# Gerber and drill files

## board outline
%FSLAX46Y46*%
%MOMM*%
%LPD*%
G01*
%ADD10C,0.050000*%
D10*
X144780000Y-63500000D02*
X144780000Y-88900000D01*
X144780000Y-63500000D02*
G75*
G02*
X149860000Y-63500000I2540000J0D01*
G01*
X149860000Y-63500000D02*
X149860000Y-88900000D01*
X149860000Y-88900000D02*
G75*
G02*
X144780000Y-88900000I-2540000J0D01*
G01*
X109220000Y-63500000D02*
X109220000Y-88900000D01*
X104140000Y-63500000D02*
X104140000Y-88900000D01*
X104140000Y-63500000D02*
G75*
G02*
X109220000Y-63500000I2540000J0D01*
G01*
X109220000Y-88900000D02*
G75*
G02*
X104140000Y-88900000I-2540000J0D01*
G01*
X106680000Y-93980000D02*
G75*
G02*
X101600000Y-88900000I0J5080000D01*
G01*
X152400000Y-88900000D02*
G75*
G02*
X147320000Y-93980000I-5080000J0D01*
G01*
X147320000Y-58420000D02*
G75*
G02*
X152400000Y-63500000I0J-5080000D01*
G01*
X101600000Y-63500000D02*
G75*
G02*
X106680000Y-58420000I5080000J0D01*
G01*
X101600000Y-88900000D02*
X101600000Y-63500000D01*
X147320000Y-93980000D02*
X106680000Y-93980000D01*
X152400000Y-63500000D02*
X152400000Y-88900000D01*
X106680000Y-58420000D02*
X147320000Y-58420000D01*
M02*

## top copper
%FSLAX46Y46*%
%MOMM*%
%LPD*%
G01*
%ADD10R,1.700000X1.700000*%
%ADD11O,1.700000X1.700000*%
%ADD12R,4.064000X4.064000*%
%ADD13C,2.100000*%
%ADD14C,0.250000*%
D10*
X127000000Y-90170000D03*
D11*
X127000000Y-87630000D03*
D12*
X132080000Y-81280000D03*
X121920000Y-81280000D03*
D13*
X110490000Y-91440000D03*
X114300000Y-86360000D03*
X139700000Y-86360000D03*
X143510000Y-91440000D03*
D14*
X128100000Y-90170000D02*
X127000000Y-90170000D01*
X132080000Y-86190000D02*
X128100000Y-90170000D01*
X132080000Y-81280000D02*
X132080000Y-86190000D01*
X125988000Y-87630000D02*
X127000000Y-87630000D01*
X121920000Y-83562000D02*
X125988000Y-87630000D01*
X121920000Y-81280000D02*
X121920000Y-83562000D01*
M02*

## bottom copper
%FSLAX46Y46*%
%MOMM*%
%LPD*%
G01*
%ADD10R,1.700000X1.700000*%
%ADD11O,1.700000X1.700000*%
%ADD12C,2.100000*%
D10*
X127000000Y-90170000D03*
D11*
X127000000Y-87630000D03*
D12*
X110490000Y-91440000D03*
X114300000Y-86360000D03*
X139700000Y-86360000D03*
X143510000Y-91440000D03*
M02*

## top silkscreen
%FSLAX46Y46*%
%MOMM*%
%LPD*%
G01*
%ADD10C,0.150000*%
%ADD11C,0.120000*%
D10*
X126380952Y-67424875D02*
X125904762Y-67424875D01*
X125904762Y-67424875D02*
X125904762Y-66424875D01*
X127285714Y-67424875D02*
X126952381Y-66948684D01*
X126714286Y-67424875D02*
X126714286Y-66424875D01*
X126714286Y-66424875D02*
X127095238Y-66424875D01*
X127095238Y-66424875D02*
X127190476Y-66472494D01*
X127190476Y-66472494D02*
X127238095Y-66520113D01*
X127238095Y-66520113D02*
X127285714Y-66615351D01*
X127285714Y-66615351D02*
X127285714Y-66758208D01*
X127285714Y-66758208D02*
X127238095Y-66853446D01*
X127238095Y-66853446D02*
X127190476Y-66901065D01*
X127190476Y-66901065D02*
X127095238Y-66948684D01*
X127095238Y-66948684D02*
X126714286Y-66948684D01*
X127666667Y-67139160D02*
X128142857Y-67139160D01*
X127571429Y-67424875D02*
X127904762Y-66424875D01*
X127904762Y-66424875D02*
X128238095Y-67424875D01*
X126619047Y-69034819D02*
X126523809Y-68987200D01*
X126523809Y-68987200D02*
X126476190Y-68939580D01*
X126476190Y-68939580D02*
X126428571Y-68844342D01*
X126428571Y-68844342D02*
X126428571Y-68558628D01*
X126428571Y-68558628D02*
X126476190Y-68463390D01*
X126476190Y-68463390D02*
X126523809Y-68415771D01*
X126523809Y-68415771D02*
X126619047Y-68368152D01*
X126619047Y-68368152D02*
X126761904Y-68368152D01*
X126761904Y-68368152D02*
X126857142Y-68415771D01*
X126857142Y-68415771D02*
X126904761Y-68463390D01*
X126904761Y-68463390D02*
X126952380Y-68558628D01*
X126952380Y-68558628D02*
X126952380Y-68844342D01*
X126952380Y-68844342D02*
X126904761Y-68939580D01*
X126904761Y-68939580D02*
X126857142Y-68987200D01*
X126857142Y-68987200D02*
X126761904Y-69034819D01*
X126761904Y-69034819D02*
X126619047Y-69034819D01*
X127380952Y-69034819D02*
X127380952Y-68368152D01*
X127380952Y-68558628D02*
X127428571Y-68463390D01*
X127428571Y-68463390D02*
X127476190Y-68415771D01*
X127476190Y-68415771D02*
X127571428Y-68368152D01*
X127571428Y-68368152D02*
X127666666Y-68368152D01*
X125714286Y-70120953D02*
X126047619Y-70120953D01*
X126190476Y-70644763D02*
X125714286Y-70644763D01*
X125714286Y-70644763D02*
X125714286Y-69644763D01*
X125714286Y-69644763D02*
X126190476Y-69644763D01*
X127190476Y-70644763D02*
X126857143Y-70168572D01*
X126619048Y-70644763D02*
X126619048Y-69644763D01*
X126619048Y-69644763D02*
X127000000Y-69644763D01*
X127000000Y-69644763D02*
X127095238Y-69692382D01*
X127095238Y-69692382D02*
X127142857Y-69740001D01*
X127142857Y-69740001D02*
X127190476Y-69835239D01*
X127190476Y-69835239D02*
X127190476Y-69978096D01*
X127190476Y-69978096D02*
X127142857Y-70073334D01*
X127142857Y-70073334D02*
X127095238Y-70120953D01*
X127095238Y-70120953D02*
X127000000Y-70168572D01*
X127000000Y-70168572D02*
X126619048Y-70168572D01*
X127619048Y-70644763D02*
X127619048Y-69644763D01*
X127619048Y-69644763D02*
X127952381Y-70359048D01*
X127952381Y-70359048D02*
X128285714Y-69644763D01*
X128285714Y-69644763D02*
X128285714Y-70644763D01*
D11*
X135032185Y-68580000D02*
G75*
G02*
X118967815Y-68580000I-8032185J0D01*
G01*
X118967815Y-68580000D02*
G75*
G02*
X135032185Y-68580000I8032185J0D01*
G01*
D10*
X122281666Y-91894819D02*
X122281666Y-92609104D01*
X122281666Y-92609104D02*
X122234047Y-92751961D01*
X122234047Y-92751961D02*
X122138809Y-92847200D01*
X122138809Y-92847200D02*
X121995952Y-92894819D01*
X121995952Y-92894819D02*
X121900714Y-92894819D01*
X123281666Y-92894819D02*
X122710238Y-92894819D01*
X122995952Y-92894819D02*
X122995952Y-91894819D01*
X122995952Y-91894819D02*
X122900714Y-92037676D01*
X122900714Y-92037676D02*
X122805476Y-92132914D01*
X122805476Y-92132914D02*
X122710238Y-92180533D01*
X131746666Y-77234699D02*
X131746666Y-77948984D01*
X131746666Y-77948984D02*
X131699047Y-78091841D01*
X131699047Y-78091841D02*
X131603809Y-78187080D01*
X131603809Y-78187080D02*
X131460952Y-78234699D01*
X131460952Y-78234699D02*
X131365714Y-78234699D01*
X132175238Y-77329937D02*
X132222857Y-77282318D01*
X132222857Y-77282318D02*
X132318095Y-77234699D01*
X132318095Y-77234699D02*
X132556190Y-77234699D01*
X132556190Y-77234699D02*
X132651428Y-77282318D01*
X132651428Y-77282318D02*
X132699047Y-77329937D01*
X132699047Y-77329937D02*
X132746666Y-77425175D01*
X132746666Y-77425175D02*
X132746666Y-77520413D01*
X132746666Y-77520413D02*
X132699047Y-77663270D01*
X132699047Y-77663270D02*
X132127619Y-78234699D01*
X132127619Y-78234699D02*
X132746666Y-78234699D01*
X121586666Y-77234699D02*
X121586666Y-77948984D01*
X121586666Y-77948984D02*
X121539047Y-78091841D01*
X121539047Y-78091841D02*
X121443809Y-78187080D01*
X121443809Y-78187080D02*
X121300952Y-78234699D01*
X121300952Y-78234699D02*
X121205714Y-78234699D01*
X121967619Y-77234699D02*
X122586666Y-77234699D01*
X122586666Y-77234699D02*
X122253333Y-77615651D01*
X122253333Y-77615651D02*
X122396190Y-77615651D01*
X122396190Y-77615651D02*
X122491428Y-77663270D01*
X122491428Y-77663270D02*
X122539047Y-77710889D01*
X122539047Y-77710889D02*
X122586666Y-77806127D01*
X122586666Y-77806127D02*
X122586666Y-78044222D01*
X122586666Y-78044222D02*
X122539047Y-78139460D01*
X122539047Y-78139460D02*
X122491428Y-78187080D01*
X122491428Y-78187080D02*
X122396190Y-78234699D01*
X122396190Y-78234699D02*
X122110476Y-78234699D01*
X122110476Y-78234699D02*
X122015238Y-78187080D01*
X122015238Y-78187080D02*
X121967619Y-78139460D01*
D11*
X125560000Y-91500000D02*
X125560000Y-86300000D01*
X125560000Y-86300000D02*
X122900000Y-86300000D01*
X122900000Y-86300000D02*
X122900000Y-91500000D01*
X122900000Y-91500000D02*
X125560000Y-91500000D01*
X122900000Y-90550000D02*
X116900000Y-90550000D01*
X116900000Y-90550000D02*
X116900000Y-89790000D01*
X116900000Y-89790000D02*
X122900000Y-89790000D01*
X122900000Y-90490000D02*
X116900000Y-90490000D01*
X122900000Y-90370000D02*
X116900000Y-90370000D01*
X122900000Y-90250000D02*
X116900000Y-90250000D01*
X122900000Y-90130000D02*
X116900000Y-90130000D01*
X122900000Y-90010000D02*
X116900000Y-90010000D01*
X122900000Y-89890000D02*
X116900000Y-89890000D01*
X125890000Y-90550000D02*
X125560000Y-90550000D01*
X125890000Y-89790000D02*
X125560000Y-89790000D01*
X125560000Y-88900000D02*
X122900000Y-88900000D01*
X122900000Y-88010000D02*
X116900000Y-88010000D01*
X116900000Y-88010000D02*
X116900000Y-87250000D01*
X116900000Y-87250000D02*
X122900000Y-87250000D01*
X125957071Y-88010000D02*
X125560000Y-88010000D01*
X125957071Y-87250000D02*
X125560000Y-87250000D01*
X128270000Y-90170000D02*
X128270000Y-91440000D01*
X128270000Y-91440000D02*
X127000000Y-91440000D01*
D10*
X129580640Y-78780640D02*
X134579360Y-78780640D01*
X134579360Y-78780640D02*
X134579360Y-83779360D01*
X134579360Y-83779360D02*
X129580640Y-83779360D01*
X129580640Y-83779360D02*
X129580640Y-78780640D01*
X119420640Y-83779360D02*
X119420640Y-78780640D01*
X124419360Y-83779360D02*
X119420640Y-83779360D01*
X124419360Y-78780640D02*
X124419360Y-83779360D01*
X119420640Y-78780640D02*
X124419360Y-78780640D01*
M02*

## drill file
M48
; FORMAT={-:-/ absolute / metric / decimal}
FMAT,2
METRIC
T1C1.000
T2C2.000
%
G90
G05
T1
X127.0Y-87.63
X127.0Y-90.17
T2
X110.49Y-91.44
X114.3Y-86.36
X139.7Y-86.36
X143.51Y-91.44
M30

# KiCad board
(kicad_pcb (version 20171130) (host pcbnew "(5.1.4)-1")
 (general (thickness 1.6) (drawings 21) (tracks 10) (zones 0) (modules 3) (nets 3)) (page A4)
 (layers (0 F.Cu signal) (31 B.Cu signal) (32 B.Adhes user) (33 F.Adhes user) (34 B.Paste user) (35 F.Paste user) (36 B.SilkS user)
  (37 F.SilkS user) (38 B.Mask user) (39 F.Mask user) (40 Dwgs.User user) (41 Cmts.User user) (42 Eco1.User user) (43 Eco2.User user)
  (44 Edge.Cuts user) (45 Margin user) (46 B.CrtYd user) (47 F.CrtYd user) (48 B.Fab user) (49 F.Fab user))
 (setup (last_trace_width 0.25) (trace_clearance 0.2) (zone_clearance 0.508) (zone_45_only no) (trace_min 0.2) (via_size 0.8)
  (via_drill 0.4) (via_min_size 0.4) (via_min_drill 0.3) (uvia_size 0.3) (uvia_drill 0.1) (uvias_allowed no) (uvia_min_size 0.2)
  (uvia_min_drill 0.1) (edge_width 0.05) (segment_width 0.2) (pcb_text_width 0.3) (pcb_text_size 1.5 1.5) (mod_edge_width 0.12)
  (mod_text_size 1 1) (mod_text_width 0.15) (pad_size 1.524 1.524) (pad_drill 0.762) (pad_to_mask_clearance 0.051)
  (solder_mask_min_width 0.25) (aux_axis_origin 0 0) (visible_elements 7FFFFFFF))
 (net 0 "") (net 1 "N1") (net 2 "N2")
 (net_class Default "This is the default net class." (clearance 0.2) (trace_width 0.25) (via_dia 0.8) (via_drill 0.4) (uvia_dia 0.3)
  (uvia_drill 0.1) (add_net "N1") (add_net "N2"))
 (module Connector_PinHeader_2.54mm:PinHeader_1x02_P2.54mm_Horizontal (layer F.Cu) (at 127 90.17 180)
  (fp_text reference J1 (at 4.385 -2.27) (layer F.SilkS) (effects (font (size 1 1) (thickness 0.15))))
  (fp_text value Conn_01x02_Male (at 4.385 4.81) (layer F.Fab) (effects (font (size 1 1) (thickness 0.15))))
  (fp_line (start 1.44 -1.33) (end 1.44 3.87) (layer F.SilkS) (width 0.12))
  (fp_line (start 1.44 3.87) (end 4.1 3.87) (layer F.SilkS) (width 0.12))
  (fp_line (start 4.1 3.87) (end 4.1 -1.33) (layer F.SilkS) (width 0.12))
  (fp_line (start 4.1 -1.33) (end 1.44 -1.33) (layer F.SilkS) (width 0.12))
  (fp_line (start 4.1 -0.38) (end 10.1 -0.38) (layer F.SilkS) (width 0.12))
  (fp_line (start 10.1 -0.38) (end 10.1 0.38) (layer F.SilkS) (width 0.12))
  (fp_line (start 10.1 0.38) (end 4.1 0.38) (layer F.SilkS) (width 0.12))
  (fp_line (start 4.1 -0.32) (end 10.1 -0.32) (layer F.SilkS) (width 0.12))
  (fp_line (start 4.1 -0.2) (end 10.1 -0.2) (layer F.SilkS) (width 0.12))
  (fp_line (start 4.1 -0.08) (end 10.1 -0.08) (layer F.SilkS) (width 0.12))
  (fp_line (start 4.1 0.04) (end 10.1 0.04) (layer F.SilkS) (width 0.12))
  (fp_line (start 4.1 0.16) (end 10.1 0.16) (layer F.SilkS) (width 0.12))
  (fp_line (start 4.1 0.28) (end 10.1 0.28) (layer F.SilkS) (width 0.12))
  (fp_line (start 1.11 -0.38) (end 1.44 -0.38) (layer F.SilkS) (width 0.12))
  (fp_line (start 1.11 0.38) (end 1.44 0.38) (layer F.SilkS) (width 0.12))
  (fp_line (start 1.44 1.27) (end 4.1 1.27) (layer F.SilkS) (width 0.12))
  (fp_line (start 4.1 2.16) (end 10.1 2.16) (layer F.SilkS) (width 0.12))
  (fp_line (start 10.1 2.16) (end 10.1 2.92) (layer F.SilkS) (width 0.12))
  (fp_line (start 10.1 2.92) (end 4.1 2.92) (layer F.SilkS) (width 0.12))
  (fp_line (start 1.042929 2.16) (end 1.44 2.16) (layer F.SilkS) (width 0.12))
  (fp_line (start 1.042929 2.92) (end 1.44 2.92) (layer F.SilkS) (width 0.12))
  (fp_line (start -1.27 0) (end -1.27 -1.27) (layer F.SilkS) (width 0.12))
  (fp_line (start -1.27 -1.27) (end 0 -1.27) (layer F.SilkS) (width 0.12))
  (pad 1 thru_hole rect (at 0 0 180) (size 1.7 1.7) (drill 1) (layers *.Cu *.Mask) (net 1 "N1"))
  (pad 2 thru_hole oval (at 0 2.54 180) (size 1.7 1.7) (drill 1) (layers *.Cu *.Mask) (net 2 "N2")))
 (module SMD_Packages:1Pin (layer F.Cu) (at 132.08 81.28)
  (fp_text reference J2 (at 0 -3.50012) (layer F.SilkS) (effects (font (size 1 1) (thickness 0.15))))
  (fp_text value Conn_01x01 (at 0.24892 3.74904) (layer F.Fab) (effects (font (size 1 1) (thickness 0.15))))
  (fp_line (start -2.49936 -2.49936) (end 2.49936 -2.49936) (layer F.SilkS) (width 0.15))
  (fp_line (start 2.49936 -2.49936) (end 2.49936 2.49936) (layer F.SilkS) (width 0.15))
  (fp_line (start 2.49936 2.49936) (end -2.49936 2.49936) (layer F.SilkS) (width 0.15))
  (fp_line (start -2.49936 2.49936) (end -2.49936 -2.49936) (layer F.SilkS) (width 0.15))
  (pad 1 smd rect (at 0 0) (size 4.064 4.064) (layers F.Cu F.Paste F.Mask) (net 1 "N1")))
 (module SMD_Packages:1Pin (layer F.Cu) (at 121.92 81.28)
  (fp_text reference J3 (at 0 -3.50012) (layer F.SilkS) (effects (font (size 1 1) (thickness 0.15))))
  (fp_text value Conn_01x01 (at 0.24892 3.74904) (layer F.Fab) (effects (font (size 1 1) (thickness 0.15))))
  (fp_line (start -2.49936 2.49936) (end -2.49936 -2.49936) (layer F.SilkS) (width 0.15))
  (fp_line (start 2.49936 2.49936) (end -2.49936 2.49936) (layer F.SilkS) (width 0.15))
  (fp_line (start 2.49936 -2.49936) (end 2.49936 2.49936) (layer F.SilkS) (width 0.15))
  (fp_line (start -2.49936 -2.49936) (end 2.49936 -2.49936) (layer F.SilkS) (width 0.15))
  (pad 1 smd rect (at 0 0) (size 4.064 4.064) (layers F.Cu F.Paste F.Mask) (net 2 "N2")))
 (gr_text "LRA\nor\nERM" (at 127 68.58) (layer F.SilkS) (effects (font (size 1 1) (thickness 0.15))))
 (gr_circle (center 127 68.58) (end 134.62 71.12) (layer F.SilkS) (width 0.12))
 (gr_line (start 144.78 63.5) (end 144.78 88.9) (layer Edge.Cuts) (width 0.05))
 (gr_arc (start 147.32 63.5) (end 149.86 63.5) (angle -180) (layer Edge.Cuts) (width 0.05))
 (gr_line (start 149.86 63.5) (end 149.86 88.9) (layer Edge.Cuts) (width 0.05))
 (gr_arc (start 147.32 88.9) (end 144.78 88.9) (angle -180) (layer Edge.Cuts) (width 0.05))
 (gr_line (start 109.22 63.5) (end 109.22 88.9) (layer Edge.Cuts) (width 0.05))
 (gr_line (start 104.14 63.5) (end 104.14 88.9) (layer Edge.Cuts) (width 0.05))
 (gr_arc (start 106.68 63.5) (end 109.22 63.5) (angle -180) (layer Edge.Cuts) (width 0.05))
 (gr_arc (start 106.68 88.9) (end 104.14 88.9) (angle -180) (layer Edge.Cuts) (width 0.05))
 (gr_arc (start 106.68 88.9) (end 101.6 88.9) (angle -90) (layer Edge.Cuts) (width 0.05))
 (gr_arc (start 147.32 88.9) (end 147.32 93.98) (angle -90) (layer Edge.Cuts) (width 0.05))
 (gr_arc (start 147.32 63.5) (end 152.4 63.5) (angle -90) (layer Edge.Cuts) (width 0.05))
 (gr_arc (start 106.68 63.5) (end 106.68 58.42) (angle -90) (layer Edge.Cuts) (width 0.05))
 (gr_line (start 101.6 88.9) (end 101.6 63.5) (layer Edge.Cuts) (width 0.05))
 (gr_line (start 147.32 93.98) (end 106.68 93.98) (layer Edge.Cuts) (width 0.05))
 (gr_line (start 152.4 63.5) (end 152.4 88.9) (layer Edge.Cuts) (width 0.05))
 (gr_line (start 106.68 58.42) (end 147.32 58.42) (layer Edge.Cuts) (width 0.05))
 (via (at 110.49 91.44) (size 2.1) (drill 2) (layers F.Cu B.Cu) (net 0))
 (via (at 114.3 86.36) (size 2.1) (drill 2) (layers F.Cu B.Cu) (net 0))
 (via (at 139.7 86.36) (size 2.1) (drill 2) (layers F.Cu B.Cu) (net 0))
 (via (at 143.51 91.44) (size 2.1) (drill 2) (layers F.Cu B.Cu) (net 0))
 (segment (start 128.1 90.17) (end 127 90.17) (width 0.25) (layer F.Cu) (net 1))
 (segment (start 132.08 86.19) (end 128.1 90.17) (width 0.25) (layer F.Cu) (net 1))
 (segment (start 132.08 81.28) (end 132.08 86.19) (width 0.25) (layer F.Cu) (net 1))
 (segment (start 125.988 87.63) (end 127 87.63) (width 0.25) (layer F.Cu) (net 2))
 (segment (start 121.92 83.562) (end 125.988 87.63) (width 0.25) (layer F.Cu) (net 2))
 (segment (start 121.92 81.28) (end 121.92 83.562) (width 0.25) (layer F.Cu) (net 2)))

